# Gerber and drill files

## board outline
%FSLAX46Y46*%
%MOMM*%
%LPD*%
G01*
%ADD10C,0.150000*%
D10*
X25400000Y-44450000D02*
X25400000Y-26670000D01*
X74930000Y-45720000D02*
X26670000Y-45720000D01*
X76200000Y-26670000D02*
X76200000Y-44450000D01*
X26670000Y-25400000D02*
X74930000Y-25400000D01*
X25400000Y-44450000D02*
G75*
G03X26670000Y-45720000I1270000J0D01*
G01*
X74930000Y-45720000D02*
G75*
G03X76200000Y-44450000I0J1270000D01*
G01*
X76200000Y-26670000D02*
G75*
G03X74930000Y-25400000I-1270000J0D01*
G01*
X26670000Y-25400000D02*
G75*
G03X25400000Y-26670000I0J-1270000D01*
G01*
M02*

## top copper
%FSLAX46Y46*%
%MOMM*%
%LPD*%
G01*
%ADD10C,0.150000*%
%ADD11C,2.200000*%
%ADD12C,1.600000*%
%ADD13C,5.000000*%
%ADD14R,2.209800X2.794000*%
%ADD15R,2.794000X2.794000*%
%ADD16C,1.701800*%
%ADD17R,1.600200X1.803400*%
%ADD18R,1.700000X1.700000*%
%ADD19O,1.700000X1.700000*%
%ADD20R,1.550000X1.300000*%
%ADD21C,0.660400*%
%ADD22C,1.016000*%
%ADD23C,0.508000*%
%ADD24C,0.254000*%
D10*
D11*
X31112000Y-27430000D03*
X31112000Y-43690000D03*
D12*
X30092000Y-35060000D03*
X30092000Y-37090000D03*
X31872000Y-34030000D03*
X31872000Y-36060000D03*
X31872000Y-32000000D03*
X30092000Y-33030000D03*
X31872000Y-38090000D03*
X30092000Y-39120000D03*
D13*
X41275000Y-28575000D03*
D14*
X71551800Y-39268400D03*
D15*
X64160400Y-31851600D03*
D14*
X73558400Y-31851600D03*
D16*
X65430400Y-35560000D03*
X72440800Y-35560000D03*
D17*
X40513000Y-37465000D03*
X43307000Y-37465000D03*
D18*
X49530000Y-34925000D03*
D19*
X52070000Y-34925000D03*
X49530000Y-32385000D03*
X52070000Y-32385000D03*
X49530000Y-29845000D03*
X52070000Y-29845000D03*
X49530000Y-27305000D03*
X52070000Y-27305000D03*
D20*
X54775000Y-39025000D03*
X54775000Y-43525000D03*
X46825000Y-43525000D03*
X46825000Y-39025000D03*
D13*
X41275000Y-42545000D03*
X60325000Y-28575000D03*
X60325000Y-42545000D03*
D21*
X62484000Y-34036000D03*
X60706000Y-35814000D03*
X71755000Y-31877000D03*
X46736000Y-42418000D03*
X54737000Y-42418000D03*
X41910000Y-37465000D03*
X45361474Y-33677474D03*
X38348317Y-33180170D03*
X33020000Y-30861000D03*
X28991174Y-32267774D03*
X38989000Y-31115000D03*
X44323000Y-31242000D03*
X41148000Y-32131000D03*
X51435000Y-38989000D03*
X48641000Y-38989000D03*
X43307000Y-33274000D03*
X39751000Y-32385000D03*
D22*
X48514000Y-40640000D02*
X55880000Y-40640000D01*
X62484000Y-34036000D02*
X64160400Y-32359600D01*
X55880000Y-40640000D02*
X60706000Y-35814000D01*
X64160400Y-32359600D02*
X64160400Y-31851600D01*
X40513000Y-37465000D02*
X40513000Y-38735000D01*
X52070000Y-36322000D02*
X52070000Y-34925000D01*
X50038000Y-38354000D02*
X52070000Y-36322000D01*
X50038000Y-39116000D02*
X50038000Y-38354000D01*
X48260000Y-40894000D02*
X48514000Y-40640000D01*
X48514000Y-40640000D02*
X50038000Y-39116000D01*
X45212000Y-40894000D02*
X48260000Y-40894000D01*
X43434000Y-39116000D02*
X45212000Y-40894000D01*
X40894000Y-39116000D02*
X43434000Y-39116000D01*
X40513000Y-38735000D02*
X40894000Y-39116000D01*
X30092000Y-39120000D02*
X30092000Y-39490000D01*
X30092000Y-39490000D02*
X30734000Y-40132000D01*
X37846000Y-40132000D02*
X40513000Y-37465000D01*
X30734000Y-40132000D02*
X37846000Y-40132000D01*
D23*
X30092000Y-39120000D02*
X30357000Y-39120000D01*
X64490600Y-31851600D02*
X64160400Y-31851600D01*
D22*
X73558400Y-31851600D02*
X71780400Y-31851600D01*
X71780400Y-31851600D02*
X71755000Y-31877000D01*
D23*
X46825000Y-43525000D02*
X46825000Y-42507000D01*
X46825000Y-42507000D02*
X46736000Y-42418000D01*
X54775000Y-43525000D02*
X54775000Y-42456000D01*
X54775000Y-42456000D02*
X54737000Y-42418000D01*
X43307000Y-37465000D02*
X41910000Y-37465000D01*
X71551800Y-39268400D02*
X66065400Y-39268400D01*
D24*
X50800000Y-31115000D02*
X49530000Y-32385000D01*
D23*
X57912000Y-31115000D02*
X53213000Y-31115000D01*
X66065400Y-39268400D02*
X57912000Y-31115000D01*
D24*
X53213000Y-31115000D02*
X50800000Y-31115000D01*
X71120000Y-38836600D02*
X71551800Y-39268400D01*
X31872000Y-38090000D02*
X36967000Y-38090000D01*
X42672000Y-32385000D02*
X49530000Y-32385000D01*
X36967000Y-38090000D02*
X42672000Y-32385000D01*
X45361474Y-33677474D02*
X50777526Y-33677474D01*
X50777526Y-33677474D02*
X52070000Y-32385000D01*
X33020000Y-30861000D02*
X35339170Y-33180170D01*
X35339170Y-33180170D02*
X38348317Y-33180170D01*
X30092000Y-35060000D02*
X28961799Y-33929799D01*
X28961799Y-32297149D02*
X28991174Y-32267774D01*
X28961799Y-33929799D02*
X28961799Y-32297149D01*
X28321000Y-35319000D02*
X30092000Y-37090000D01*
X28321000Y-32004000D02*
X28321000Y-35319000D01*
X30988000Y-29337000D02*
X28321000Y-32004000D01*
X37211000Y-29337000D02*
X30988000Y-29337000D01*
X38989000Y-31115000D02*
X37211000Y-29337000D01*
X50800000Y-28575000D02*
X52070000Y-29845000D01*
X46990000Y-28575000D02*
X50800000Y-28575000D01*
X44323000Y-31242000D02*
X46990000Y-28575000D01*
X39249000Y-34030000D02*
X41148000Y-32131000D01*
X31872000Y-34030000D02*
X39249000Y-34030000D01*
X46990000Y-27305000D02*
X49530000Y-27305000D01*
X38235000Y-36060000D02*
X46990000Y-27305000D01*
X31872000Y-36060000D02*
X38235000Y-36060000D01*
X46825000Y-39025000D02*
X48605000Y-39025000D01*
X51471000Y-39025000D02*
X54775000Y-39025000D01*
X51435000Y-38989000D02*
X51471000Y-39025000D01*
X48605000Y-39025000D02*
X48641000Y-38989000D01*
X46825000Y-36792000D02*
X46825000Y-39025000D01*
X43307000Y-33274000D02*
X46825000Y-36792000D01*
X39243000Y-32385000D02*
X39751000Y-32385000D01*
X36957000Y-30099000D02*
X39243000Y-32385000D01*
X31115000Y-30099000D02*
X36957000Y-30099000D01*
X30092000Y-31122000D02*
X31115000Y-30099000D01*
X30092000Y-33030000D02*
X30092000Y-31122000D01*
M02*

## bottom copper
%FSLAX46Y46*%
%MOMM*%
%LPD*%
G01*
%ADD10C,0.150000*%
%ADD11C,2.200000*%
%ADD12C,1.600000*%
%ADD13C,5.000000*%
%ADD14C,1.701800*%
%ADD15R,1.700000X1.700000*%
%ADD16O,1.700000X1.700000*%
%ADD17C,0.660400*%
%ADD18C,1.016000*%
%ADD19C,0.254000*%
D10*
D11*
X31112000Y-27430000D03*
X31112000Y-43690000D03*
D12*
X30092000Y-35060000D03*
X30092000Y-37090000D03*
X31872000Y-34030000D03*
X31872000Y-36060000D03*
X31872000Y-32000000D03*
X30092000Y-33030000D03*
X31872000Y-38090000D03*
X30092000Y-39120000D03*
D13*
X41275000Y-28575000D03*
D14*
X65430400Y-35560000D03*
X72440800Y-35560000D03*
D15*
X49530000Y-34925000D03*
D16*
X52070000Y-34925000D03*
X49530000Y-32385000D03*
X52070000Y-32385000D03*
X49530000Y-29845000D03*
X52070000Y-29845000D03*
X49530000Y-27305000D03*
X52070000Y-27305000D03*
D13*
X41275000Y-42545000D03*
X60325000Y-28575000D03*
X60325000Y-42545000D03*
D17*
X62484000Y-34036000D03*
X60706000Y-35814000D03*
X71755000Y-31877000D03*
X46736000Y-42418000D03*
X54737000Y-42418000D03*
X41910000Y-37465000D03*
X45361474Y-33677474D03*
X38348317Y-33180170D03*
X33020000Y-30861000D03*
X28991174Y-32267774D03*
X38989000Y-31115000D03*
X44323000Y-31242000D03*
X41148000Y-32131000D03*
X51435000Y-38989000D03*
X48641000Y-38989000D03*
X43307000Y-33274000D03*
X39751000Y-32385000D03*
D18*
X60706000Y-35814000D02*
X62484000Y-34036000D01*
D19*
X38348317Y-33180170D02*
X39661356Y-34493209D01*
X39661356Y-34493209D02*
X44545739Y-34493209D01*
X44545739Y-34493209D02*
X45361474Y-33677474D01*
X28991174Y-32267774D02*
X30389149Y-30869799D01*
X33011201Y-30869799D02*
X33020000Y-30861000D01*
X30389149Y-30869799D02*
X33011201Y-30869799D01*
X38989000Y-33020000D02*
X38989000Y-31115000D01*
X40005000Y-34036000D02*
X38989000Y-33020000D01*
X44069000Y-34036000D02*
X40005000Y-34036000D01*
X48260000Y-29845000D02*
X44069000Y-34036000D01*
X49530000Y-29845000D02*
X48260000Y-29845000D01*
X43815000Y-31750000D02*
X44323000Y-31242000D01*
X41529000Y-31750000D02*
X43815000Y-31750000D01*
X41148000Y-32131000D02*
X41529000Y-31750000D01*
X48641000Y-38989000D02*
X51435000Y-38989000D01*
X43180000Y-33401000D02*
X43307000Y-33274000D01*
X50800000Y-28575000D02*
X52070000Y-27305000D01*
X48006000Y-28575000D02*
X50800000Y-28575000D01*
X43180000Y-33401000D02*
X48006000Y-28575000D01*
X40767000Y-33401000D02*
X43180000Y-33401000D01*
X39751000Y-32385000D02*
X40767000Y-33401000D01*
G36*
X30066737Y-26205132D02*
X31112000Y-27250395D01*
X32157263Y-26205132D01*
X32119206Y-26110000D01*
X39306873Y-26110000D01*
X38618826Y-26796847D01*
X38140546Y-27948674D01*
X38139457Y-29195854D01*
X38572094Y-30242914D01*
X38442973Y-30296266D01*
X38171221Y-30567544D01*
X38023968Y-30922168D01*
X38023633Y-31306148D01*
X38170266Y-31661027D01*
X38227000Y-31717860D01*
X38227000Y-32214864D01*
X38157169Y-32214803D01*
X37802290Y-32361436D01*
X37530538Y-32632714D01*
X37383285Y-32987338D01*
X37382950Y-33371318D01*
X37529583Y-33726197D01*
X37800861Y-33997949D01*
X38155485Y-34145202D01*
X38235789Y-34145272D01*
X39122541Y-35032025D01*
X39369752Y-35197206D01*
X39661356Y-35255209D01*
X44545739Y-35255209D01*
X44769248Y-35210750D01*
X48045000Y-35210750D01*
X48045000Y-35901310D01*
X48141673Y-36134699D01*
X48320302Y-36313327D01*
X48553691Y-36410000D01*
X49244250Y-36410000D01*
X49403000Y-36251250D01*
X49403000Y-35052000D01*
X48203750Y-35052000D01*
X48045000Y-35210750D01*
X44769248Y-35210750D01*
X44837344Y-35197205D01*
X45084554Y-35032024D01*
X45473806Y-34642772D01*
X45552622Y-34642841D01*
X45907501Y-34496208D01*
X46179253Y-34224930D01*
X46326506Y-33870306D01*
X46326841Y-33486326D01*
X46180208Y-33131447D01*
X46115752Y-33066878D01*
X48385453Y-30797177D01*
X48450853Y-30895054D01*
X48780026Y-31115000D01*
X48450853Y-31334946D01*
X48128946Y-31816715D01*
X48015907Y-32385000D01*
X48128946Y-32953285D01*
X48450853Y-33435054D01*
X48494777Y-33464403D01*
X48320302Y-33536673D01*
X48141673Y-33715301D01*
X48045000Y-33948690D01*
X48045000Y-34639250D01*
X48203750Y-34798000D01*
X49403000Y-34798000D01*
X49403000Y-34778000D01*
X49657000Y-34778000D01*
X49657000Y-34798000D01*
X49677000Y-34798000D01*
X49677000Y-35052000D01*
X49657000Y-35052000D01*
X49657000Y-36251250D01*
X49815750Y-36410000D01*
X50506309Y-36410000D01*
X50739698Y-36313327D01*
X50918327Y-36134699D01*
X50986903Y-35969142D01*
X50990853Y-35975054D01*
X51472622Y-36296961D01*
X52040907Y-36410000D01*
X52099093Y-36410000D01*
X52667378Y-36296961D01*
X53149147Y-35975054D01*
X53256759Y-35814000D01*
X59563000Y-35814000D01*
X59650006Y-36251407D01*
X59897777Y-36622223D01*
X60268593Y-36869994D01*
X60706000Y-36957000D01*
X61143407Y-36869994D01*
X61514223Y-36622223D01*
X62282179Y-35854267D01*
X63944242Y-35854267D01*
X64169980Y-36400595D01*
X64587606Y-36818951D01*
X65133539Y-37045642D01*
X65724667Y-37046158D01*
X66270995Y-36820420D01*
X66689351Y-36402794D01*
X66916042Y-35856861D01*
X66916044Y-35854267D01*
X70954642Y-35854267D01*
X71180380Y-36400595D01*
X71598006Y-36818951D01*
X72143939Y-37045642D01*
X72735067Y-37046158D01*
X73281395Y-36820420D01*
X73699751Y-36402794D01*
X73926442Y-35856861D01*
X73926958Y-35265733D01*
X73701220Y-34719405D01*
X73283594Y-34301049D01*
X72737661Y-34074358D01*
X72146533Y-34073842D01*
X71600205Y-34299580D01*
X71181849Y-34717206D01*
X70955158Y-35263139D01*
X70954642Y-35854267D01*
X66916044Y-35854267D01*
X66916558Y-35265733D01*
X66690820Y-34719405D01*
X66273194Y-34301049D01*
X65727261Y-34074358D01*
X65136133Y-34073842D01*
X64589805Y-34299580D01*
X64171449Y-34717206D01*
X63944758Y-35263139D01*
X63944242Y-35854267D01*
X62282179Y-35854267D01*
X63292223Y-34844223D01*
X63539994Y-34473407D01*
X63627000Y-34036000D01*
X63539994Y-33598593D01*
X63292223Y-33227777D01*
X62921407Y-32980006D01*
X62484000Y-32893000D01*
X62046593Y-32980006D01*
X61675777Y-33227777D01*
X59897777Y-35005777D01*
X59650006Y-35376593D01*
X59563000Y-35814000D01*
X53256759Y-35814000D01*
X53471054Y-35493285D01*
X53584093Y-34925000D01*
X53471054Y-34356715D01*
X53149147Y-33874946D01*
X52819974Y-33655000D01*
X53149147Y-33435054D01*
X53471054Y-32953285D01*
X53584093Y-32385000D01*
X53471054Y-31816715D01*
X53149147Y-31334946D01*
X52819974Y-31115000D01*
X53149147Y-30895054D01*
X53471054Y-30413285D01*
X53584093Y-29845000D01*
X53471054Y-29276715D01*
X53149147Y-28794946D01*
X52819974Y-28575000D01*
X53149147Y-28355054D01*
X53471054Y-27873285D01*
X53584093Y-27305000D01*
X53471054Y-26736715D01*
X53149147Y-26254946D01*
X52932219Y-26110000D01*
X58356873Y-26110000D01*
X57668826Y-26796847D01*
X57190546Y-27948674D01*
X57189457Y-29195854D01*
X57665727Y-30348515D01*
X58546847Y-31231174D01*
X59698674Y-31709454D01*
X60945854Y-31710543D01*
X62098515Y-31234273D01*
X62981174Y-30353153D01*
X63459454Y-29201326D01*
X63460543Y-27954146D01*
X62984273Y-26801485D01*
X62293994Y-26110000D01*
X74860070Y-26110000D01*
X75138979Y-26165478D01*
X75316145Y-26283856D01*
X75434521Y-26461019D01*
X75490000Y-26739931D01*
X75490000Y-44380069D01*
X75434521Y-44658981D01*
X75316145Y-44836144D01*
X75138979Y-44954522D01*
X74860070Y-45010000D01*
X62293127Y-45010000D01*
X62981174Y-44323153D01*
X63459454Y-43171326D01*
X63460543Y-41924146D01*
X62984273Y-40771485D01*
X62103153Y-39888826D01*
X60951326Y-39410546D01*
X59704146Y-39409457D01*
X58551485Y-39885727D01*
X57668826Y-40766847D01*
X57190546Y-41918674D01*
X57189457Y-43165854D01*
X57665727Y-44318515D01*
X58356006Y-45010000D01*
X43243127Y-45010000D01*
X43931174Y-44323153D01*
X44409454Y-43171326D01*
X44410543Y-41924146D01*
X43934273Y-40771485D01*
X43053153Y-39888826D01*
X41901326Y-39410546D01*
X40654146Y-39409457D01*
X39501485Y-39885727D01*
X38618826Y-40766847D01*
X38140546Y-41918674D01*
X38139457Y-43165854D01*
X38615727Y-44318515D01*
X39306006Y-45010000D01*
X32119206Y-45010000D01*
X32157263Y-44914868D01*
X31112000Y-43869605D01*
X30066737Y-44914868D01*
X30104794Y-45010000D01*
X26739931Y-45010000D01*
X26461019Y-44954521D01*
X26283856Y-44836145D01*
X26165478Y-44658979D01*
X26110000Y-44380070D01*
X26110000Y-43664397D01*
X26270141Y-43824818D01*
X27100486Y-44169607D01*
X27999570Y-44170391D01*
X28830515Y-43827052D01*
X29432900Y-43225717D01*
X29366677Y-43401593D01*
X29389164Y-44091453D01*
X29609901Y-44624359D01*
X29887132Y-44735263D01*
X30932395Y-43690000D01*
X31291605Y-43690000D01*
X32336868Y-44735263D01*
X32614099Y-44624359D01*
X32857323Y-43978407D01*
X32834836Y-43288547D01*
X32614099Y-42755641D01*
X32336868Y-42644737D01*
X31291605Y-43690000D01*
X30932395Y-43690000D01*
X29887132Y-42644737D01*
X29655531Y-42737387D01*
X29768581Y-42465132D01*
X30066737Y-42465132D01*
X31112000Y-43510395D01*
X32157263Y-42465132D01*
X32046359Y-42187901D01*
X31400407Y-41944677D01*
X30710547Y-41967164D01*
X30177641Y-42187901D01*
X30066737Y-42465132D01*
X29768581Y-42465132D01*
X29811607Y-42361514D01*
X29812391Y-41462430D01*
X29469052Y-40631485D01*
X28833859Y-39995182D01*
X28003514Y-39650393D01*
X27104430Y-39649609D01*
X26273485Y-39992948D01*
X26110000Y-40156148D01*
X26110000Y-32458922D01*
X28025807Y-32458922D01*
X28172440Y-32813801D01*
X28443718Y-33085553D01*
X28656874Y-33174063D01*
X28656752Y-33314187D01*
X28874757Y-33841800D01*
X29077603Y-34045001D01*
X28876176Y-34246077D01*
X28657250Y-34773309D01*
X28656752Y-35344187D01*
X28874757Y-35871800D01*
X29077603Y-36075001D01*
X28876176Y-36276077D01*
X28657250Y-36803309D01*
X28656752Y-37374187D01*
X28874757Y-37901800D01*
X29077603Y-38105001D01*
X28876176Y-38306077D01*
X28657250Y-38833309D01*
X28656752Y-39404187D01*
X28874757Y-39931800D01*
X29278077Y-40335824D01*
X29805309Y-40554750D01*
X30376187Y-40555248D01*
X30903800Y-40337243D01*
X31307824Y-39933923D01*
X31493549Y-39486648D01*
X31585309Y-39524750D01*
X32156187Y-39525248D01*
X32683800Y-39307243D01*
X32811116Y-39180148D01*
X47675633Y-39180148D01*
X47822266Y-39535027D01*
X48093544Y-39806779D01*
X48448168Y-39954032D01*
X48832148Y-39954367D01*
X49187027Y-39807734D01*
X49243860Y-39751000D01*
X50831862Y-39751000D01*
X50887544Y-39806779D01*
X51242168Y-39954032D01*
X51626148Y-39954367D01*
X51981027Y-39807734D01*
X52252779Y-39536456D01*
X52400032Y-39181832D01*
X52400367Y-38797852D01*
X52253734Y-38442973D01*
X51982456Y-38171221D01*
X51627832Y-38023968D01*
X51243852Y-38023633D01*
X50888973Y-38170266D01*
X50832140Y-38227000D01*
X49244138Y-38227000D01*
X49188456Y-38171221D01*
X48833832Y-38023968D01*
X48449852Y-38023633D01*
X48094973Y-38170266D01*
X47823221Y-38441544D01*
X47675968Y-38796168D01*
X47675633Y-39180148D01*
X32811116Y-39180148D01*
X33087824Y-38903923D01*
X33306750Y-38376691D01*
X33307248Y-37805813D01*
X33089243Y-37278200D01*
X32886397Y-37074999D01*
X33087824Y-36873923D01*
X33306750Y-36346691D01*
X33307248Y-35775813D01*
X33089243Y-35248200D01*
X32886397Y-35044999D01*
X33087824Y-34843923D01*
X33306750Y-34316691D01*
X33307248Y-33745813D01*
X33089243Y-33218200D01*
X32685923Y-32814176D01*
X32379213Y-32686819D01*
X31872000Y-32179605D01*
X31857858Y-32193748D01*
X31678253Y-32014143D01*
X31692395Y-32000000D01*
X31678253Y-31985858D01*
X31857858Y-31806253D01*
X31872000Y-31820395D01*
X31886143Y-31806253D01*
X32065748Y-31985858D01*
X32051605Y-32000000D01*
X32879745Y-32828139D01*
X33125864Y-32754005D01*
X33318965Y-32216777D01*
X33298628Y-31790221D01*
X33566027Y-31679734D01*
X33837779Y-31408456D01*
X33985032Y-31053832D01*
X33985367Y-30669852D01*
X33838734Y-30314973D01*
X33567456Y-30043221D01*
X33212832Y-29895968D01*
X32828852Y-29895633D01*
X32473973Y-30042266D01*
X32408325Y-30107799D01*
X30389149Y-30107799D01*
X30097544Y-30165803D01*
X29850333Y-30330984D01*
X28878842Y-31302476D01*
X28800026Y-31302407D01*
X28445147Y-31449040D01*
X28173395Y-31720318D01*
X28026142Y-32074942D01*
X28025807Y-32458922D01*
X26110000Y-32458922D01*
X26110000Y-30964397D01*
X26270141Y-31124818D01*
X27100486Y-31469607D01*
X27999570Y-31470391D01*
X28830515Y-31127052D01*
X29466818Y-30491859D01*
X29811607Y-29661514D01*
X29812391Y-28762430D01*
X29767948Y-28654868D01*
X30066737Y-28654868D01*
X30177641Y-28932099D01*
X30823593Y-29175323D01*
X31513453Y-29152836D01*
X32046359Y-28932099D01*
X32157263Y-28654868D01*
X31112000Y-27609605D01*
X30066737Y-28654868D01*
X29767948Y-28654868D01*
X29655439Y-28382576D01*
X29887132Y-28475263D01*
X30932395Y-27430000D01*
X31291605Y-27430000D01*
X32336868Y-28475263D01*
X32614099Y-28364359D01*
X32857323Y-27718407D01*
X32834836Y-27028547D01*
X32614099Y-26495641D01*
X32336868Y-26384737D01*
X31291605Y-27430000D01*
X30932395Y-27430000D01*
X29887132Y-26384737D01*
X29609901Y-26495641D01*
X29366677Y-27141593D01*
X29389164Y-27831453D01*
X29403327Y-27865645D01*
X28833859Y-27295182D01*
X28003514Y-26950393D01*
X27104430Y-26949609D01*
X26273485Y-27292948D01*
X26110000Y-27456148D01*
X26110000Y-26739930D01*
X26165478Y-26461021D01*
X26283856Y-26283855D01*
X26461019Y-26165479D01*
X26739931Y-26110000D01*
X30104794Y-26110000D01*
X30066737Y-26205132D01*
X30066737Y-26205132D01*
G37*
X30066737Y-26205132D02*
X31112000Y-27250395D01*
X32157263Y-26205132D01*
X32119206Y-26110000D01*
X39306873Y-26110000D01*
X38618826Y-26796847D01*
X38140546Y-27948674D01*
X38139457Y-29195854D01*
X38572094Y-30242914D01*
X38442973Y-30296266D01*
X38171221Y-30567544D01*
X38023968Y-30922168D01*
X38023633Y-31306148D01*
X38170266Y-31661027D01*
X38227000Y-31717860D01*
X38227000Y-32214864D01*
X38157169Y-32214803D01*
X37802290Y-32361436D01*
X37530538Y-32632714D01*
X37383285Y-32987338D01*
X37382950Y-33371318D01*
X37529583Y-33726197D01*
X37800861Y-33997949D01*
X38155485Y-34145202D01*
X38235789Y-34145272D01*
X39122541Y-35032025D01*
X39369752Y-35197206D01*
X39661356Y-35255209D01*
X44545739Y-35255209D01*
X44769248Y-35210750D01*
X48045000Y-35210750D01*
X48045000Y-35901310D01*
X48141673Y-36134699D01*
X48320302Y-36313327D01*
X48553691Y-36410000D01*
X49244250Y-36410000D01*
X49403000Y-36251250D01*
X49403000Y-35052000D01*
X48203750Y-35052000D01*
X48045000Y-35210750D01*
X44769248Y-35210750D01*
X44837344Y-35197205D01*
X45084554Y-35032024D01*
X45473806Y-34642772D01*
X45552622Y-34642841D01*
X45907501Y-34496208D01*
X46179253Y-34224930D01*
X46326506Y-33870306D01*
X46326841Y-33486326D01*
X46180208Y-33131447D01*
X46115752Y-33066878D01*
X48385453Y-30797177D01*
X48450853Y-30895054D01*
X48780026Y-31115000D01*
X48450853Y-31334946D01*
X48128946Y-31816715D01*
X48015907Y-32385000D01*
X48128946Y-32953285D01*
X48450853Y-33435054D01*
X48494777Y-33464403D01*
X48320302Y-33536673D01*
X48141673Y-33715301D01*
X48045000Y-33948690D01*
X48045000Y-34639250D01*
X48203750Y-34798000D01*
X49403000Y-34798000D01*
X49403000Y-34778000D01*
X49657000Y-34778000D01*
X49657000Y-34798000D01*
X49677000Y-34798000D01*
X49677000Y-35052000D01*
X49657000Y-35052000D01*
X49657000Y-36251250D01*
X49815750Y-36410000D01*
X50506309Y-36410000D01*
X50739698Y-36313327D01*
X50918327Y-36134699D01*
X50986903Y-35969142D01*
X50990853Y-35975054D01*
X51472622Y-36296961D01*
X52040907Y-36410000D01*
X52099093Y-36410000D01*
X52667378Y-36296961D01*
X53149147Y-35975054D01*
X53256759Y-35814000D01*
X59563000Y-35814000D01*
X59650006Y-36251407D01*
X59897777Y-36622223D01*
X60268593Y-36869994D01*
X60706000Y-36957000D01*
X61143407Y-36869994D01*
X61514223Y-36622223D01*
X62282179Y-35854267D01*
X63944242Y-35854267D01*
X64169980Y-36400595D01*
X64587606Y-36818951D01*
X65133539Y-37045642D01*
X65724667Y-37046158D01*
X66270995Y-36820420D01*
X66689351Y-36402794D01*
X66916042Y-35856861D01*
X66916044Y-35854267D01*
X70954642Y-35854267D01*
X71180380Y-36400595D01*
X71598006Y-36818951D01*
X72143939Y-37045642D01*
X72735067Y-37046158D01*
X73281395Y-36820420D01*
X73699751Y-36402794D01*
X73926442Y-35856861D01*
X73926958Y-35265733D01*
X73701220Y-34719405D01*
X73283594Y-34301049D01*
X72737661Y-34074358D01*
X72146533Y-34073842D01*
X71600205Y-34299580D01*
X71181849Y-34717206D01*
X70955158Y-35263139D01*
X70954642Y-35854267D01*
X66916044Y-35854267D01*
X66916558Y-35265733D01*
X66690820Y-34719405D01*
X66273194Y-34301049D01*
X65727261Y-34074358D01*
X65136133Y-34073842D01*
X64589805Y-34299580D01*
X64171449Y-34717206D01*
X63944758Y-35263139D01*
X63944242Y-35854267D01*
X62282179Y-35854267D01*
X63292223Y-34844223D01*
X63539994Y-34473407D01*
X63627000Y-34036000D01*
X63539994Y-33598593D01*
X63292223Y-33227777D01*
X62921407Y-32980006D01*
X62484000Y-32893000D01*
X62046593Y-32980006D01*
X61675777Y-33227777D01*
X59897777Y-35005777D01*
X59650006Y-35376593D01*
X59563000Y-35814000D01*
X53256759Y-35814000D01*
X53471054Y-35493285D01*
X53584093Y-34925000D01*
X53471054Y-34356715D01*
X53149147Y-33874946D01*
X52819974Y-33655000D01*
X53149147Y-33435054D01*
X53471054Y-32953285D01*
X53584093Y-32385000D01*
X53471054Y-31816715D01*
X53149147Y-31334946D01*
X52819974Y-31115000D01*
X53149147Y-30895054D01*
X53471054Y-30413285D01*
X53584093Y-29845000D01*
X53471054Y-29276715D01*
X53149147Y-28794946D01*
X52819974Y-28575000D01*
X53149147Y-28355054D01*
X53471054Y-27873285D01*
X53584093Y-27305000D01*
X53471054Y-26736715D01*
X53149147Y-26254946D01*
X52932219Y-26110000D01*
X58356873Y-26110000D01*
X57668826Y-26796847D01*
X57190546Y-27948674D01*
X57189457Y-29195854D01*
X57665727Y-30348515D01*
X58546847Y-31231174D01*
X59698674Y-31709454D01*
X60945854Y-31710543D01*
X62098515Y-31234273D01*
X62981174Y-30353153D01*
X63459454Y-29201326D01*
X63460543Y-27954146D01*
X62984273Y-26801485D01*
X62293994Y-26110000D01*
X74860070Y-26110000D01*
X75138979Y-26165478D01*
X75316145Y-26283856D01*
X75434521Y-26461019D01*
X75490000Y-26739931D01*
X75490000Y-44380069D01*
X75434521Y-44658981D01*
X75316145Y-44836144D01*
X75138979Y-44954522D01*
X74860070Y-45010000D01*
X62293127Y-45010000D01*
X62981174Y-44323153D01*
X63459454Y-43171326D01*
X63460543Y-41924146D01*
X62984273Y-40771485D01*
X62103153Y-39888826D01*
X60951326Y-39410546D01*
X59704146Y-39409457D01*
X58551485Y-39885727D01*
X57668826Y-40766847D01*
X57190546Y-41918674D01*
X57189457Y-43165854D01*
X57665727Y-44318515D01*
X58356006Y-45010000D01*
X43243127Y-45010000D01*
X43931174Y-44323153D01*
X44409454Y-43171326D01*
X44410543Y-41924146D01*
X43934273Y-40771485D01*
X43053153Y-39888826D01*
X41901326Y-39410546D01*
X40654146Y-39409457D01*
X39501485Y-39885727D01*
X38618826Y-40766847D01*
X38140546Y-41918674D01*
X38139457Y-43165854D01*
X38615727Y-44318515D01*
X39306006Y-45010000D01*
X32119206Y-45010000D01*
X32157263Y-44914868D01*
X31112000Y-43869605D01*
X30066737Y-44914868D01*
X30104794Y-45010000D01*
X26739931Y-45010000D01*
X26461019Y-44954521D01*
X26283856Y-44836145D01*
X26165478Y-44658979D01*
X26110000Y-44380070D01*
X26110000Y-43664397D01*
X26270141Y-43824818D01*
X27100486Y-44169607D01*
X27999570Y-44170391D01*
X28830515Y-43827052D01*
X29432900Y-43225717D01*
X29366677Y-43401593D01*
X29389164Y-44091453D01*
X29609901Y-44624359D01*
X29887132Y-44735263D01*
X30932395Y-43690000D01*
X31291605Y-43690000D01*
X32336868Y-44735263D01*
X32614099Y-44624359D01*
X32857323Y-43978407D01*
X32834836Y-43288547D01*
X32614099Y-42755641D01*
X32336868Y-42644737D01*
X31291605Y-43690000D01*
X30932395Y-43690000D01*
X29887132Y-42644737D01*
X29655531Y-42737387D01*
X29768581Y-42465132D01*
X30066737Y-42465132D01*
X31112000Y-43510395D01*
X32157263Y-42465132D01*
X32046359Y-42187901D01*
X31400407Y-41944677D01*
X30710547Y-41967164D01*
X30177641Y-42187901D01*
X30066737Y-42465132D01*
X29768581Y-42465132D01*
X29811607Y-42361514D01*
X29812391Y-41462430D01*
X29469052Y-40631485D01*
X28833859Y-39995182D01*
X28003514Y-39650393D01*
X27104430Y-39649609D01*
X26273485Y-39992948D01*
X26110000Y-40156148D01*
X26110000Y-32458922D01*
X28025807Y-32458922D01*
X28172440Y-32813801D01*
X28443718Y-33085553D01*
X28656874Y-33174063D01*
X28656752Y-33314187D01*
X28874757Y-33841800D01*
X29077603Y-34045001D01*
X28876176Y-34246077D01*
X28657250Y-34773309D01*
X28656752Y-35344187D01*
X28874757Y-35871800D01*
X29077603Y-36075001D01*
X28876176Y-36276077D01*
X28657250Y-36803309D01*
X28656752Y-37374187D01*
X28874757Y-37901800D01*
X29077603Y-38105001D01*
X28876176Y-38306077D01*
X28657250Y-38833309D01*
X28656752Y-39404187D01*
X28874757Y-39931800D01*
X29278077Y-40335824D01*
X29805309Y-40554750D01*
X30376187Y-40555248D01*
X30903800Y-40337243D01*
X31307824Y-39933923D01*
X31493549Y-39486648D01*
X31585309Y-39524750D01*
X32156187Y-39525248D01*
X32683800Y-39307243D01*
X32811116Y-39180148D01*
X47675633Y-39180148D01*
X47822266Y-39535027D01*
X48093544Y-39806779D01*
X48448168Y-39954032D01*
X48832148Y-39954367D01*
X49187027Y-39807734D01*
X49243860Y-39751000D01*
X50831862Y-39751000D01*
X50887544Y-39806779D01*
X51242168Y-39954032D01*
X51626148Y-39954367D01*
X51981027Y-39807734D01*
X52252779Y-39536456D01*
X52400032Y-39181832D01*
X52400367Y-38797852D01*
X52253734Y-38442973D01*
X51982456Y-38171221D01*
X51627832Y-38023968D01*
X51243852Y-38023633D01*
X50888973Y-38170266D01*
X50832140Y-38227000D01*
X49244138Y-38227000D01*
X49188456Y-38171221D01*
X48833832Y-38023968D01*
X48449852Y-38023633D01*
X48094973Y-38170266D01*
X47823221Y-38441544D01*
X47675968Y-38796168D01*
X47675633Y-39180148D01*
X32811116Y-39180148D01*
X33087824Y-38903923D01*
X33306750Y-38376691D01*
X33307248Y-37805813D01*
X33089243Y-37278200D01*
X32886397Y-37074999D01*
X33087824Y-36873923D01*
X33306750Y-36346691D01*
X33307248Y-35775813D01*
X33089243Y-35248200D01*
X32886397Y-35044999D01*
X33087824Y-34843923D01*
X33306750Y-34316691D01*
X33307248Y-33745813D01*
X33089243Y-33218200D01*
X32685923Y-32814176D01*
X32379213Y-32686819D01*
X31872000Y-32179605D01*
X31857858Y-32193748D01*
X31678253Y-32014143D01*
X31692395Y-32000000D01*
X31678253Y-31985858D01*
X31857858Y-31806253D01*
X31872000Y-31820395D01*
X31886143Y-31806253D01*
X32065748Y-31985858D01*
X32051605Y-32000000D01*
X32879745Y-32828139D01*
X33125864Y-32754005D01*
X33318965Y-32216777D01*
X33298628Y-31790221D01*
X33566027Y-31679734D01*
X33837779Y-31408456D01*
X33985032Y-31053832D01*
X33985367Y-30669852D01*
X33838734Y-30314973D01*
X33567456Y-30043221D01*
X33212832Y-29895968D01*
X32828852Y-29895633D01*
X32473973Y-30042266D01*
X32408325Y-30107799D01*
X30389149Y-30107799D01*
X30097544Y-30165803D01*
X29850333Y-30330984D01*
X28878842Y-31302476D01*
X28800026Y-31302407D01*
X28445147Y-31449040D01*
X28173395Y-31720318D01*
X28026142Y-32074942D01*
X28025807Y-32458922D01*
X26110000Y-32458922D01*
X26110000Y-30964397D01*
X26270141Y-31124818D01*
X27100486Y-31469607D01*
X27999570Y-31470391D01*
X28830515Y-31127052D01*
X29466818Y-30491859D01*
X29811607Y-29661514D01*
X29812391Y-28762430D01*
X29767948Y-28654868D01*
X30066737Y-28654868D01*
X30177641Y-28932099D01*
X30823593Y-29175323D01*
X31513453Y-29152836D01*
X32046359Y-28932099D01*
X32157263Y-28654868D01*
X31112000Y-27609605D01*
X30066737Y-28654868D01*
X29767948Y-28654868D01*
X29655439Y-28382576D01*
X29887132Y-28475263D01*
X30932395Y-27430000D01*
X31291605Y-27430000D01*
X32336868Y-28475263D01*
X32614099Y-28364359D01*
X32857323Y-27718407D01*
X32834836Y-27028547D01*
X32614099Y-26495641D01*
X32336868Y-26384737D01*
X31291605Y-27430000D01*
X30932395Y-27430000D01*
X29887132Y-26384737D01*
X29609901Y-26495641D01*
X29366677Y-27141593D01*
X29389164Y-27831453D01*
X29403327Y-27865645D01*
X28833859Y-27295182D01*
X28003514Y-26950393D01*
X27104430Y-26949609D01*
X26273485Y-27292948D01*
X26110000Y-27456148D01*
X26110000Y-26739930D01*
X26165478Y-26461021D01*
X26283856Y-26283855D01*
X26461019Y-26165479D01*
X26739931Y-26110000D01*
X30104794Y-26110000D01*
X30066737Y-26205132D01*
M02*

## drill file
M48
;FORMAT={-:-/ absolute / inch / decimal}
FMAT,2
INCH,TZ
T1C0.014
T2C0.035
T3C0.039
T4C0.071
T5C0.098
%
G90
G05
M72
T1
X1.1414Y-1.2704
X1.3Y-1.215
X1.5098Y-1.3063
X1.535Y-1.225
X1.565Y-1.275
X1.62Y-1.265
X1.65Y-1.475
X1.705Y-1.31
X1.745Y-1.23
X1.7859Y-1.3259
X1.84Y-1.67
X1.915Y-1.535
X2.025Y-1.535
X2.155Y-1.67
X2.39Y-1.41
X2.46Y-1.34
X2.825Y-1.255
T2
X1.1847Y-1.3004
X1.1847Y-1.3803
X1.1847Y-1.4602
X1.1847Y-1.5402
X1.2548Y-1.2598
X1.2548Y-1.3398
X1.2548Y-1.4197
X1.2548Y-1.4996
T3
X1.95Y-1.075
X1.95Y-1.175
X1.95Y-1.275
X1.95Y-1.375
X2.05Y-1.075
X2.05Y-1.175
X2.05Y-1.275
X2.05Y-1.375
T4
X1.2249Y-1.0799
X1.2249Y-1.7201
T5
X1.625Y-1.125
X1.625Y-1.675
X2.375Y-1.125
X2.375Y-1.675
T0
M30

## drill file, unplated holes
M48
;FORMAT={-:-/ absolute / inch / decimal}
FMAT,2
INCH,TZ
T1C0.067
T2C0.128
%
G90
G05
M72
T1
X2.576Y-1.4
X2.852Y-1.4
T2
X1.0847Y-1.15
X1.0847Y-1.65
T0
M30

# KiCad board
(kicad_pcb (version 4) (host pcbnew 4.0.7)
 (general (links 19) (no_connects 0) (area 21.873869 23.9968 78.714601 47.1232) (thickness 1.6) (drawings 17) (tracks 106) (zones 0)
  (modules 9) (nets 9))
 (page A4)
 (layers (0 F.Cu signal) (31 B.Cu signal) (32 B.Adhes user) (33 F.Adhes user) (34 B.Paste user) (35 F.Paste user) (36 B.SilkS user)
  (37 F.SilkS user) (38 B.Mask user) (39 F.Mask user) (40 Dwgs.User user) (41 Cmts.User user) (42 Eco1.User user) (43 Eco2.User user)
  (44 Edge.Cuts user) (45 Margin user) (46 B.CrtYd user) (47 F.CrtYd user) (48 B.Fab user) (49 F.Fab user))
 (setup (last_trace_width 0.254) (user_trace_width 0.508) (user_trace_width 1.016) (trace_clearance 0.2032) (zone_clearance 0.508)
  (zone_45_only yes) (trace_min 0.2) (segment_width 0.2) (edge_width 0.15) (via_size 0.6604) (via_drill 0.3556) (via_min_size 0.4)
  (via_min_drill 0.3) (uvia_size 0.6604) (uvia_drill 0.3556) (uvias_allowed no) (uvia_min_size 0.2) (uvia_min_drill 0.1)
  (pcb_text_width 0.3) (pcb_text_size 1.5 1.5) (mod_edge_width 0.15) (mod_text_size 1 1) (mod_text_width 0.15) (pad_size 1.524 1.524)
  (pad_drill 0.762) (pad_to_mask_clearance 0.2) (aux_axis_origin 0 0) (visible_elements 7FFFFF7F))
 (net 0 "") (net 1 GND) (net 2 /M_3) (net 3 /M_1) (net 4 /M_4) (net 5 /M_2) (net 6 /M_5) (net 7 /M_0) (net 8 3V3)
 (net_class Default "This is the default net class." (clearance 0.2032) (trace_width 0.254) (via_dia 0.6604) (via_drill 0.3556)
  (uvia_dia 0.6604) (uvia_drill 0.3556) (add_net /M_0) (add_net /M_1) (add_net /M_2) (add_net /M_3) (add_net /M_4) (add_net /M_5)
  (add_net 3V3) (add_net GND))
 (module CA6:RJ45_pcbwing (layer F.Cu) (at 29.972 35.56 270)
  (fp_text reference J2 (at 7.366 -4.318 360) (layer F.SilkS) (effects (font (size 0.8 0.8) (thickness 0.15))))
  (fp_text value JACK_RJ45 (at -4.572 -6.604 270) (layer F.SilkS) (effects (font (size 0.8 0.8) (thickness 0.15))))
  (pad 8 thru_hole circle (at -8.13 -1.14 270) (size 2.2 2.2) (drill 1.8) (layers *.Cu *.Mask F.SilkS) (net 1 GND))
  (pad 8 thru_hole circle (at 8.13 -1.14 270) (size 2.2 2.2) (drill 1.8) (layers *.Cu *.Mask F.SilkS) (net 1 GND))
  (pad "" np_thru_hole circle (at -6.35 2.42 270) (size 3.25 3.25) (drill 3.25) (layers *.Cu *.Mask F.SilkS))
  (pad "" np_thru_hole circle (at 6.35 2.42 270) (size 3.25 3.25) (drill 3.25) (layers *.Cu *.Mask F.SilkS))
  (pad 5 thru_hole circle (at -0.5 -0.12 270) (size 1.6 1.6) (drill 0.89) (layers *.Cu *.Mask F.SilkS) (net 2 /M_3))
  (pad 3 thru_hole circle (at 1.53 -0.12 270) (size 1.6 1.6) (drill 0.89) (layers *.Cu *.Mask F.SilkS) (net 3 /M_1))
  (pad 6 thru_hole circle (at -1.53 -1.9 270) (size 1.6 1.6) (drill 0.89) (layers *.Cu *.Mask F.SilkS) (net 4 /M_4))
  (pad 4 thru_hole circle (at 0.5 -1.9 270) (size 1.6 1.6) (drill 0.89) (layers *.Cu *.Mask F.SilkS) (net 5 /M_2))
  (pad 8 thru_hole circle (at -3.56 -1.9 270) (size 1.6 1.6) (drill 0.89) (layers *.Cu *.Mask F.SilkS) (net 1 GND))
  (pad 7 thru_hole circle (at -2.53 -0.12 270) (size 1.6 1.6) (drill 0.89) (layers *.Cu *.Mask F.SilkS) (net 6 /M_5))
  (pad 2 thru_hole circle (at 2.53 -1.9 270) (size 1.6 1.6) (drill 0.89) (layers *.Cu *.Mask F.SilkS) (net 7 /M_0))
  (pad 1 thru_hole circle (at 3.56 -0.12 270) (size 1.6 1.6) (drill 0.89) (layers *.Cu *.Mask F.SilkS) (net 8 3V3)))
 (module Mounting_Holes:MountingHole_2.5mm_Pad (layer F.Cu) (at 41.275 28.575)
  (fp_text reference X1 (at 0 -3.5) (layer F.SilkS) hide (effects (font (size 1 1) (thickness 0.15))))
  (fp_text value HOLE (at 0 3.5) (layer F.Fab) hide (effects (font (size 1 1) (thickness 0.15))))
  (pad 1 thru_hole circle (at 0 0) (size 5 5) (drill 2.5) (layers *.Cu *.Mask)))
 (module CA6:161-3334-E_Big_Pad (layer F.Cu) (at 75.946 35.56 180)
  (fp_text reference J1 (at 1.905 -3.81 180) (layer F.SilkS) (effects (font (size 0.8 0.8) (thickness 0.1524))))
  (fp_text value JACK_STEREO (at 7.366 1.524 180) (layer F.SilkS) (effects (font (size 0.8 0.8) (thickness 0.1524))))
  (pad 1 smd rect (at 4.3942 -3.7084 180) (size 2.2098 2.794) (layers F.Cu F.Paste F.Mask) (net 7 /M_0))
  (pad 2 smd rect (at 11.7856 3.7084 180) (size 2.794 2.794) (layers F.Cu F.Paste F.Mask) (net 8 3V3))
  (pad 3 smd rect (at 2.3876 3.7084 180) (size 2.2098 2.794) (layers F.Cu F.Paste F.Mask) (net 1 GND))
  (pad "" np_thru_hole circle (at 10.5156 0 90) (size 1.7018 1.7018) (drill 1.7) (layers *.Cu *.Mask F.SilkS))
  (pad "" np_thru_hole circle (at 3.5052 0 90) (size 1.7018 1.7018) (drill 1.7) (layers *.Cu *.Mask F.SilkS)))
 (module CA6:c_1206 (layer F.Cu) (at 41.91 37.465 180)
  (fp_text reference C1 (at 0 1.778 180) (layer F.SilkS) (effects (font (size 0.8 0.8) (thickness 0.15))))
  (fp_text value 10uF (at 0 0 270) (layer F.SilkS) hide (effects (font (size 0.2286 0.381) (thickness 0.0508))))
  (pad 1 smd rect (at 1.397 0 180) (size 1.6002 1.8034) (layers F.Cu F.Paste F.Mask) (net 8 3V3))
  (pad 2 smd rect (at -1.397 0 180) (size 1.6002 1.8034) (layers F.Cu F.Paste F.Mask) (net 1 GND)))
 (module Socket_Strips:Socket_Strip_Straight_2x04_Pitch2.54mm (layer F.Cu) (at 49.53 34.925 180)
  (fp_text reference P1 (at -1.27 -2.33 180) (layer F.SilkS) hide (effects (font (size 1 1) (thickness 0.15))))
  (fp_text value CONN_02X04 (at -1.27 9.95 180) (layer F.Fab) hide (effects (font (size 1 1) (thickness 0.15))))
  (pad 1 thru_hole rect (at 0 0 180) (size 1.7 1.7) (drill 1) (layers *.Cu *.Mask) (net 1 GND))
  (pad 2 thru_hole oval (at -2.54 0 180) (size 1.7 1.7) (drill 1) (layers *.Cu *.Mask) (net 8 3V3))
  (pad 3 thru_hole oval (at 0 2.54 180) (size 1.7 1.7) (drill 1) (layers *.Cu *.Mask) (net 7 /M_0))
  (pad 4 thru_hole oval (at -2.54 2.54 180) (size 1.7 1.7) (drill 1) (layers *.Cu *.Mask) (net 2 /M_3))
  (pad 5 thru_hole oval (at 0 5.08 180) (size 1.7 1.7) (drill 1) (layers *.Cu *.Mask) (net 3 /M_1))
  (pad 6 thru_hole oval (at -2.54 5.08 180) (size 1.7 1.7) (drill 1) (layers *.Cu *.Mask) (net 4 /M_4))
  (pad 7 thru_hole oval (at 0 7.62 180) (size 1.7 1.7) (drill 1) (layers *.Cu *.Mask) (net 5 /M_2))
  (pad 8 thru_hole oval (at -2.54 7.62 180) (size 1.7 1.7) (drill 1) (layers *.Cu *.Mask) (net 6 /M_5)))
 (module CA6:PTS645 (layer F.Cu) (at 50.8 41.275 180)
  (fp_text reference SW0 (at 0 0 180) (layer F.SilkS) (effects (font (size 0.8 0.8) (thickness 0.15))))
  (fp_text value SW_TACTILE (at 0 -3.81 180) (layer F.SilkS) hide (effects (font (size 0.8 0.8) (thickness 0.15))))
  (pad 3 smd rect (at -3.975 2.25 180) (size 1.55 1.3) (layers F.Cu F.Paste F.Mask) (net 6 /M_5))
  (pad 1 smd rect (at -3.975 -2.25 180) (size 1.55 1.3) (layers F.Cu F.Paste F.Mask) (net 1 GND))
  (pad 2 smd rect (at 3.975 -2.25 180) (size 1.55 1.3) (layers F.Cu F.Paste F.Mask) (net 1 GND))
  (pad 4 smd rect (at 3.975 2.25 180) (size 1.55 1.3) (layers F.Cu F.Paste F.Mask) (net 6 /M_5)))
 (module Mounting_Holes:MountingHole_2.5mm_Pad (layer F.Cu) (at 41.275 42.545)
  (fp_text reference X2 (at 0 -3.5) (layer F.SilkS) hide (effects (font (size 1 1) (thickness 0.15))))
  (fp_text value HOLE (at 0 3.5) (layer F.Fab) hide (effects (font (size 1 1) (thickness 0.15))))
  (pad 1 thru_hole circle (at 0 0) (size 5 5) (drill 2.5) (layers *.Cu *.Mask)))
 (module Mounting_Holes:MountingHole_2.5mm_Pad (layer F.Cu) (at 60.325 28.575)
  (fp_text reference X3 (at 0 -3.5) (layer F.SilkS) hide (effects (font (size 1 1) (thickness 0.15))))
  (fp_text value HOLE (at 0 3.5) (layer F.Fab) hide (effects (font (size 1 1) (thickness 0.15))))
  (pad 1 thru_hole circle (at 0 0) (size 5 5) (drill 2.5) (layers *.Cu *.Mask)))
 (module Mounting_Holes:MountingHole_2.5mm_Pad (layer F.Cu) (at 60.325 42.545)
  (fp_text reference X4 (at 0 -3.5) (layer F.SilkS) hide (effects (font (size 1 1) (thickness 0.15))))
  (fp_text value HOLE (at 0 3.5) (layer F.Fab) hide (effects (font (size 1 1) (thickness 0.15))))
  (pad 1 thru_hole circle (at 0 0) (size 5 5) (drill 2.5) (layers *.Cu *.Mask)))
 (gr_line (start 25.4 44.45) (end 25.4 26.67) (angle 90) (layer Edge.Cuts) (width 0.15))
 (gr_line (start 74.93 45.72) (end 26.67 45.72) (angle 90) (layer Edge.Cuts) (width 0.15))
 (gr_line (start 76.2 26.67) (end 76.2 44.45) (angle 90) (layer Edge.Cuts) (width 0.15))
 (gr_line (start 26.67 25.4) (end 74.93 25.4) (angle 90) (layer Edge.Cuts) (width 0.15))
 (gr_arc (start 26.67 44.45) (end 26.67 45.72) (angle 90) (layer Edge.Cuts) (width 0.15))
 (gr_arc (start 74.93 44.45) (end 76.2 44.45) (angle 90) (layer Edge.Cuts) (width 0.15))
 (gr_arc (start 74.93 26.67) (end 74.93 25.4) (angle 90) (layer Edge.Cuts) (width 0.15))
 (gr_arc (start 26.67 26.67) (end 25.4 26.67) (angle 90) (layer Edge.Cuts) (width 0.15))
 (segment (start 48.514 40.64) (end 55.88 40.64) (width 1.016) (layer F.Cu) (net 8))
 (segment (start 62.484 34.036) (end 64.1604 32.3596) (width 1.016) (layer F.Cu) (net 8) (status 20))
 (via (at 62.484 34.036) (size 0.6604) (drill 0.3556) (layers F.Cu B.Cu) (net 8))
 (segment (start 60.706 35.814) (end 62.484 34.036) (width 1.016) (layer B.Cu) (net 8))
 (via (at 60.706 35.814) (size 0.6604) (drill 0.3556) (layers F.Cu B.Cu) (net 8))
 (segment (start 55.88 40.64) (end 60.706 35.814) (width 1.016) (layer F.Cu) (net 8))
 (segment (start 64.1604 32.3596) (end 64.1604 31.8516) (width 1.016) (layer F.Cu) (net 8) (status 30))
 (segment (start 40.513 37.465) (end 40.513 38.735) (width 1.016) (layer F.Cu) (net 8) (status 10))
 (segment (start 52.07 36.322) (end 52.07 34.925) (width 1.016) (layer F.Cu) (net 8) (status 20))
 (segment (start 50.038 38.354) (end 52.07 36.322) (width 1.016) (layer F.Cu) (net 8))
 (segment (start 50.038 39.116) (end 50.038 38.354) (width 1.016) (layer F.Cu) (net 8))
 (segment (start 48.26 40.894) (end 48.514 40.64) (width 1.016) (layer F.Cu) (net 8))
 (segment (start 48.514 40.64) (end 50.038 39.116) (width 1.016) (layer F.Cu) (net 8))
 (segment (start 45.212 40.894) (end 48.26 40.894) (width 1.016) (layer F.Cu) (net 8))
 (segment (start 43.434 39.116) (end 45.212 40.894) (width 1.016) (layer F.Cu) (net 8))
 (segment (start 40.894 39.116) (end 43.434 39.116) (width 1.016) (layer F.Cu) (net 8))
 (segment (start 40.513 38.735) (end 40.894 39.116) (width 1.016) (layer F.Cu) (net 8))
 (segment (start 30.092 39.12) (end 30.092 39.49) (width 1.016) (layer F.Cu) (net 8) (status 30))
 (segment (start 30.092 39.49) (end 30.734 40.132) (width 1.016) (layer F.Cu) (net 8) (status 10))
 (segment (start 37.846 40.132) (end 40.513 37.465) (width 1.016) (layer F.Cu) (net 8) (status 20))
 (segment (start 30.734 40.132) (end 37.846 40.132) (width 1.016) (layer F.Cu) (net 8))
 (segment (start 30.092 39.12) (end 30.357 39.12) (width 0.508) (layer F.Cu) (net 8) (status 30))
 (segment (start 64.4906 31.8516) (end 64.1604 31.8516) (width 0.508) (layer F.Cu) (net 8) (status 30))
 (segment (start 73.5584 31.8516) (end 71.7804 31.8516) (width 1.016) (layer F.Cu) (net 1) (status 10))
 (via (at 71.755 31.877) (size 0.6604) (drill 0.3556) (layers F.Cu B.Cu) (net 1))
 (segment (start 71.7804 31.8516) (end 71.755 31.877) (width 1.016) (layer F.Cu) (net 1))
 (segment (start 46.825 43.525) (end 46.825 42.507) (width 0.508) (layer F.Cu) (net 1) (status 10))
 (via (at 46.736 42.418) (size 0.6604) (drill 0.3556) (layers F.Cu B.Cu) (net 1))
 (segment (start 46.825 42.507) (end 46.736 42.418) (width 0.508) (layer F.Cu) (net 1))
 (segment (start 54.775 43.525) (end 54.775 42.456) (width 0.508) (layer F.Cu) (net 1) (status 10))
 (via (at 54.737 42.418) (size 0.6604) (drill 0.3556) (layers F.Cu B.Cu) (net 1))
 (segment (start 54.775 42.456) (end 54.737 42.418) (width 0.508) (layer F.Cu) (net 1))
 (segment (start 43.307 37.465) (end 41.91 37.465) (width 0.508) (layer F.Cu) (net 1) (status 10))
 (via (at 41.91 37.465) (size 0.6604) (drill 0.3556) (layers F.Cu B.Cu) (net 1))
 (segment (start 71.5518 39.2684) (end 66.0654 39.2684) (width 0.508) (layer F.Cu) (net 7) (status 10))
 (segment (start 50.8 31.115) (end 49.53 32.385) (width 0.254) (layer F.Cu) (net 7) (status 20))
 (segment (start 57.912 31.115) (end 53.213 31.115) (width 0.508) (layer F.Cu) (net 7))
 (segment (start 66.0654 39.2684) (end 57.912 31.115) (width 0.508) (layer F.Cu) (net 7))
 (segment (start 53.213 31.115) (end 50.8 31.115) (width 0.254) (layer F.Cu) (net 7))
 (segment (start 71.12 38.8366) (end 71.5518 39.2684) (width 0.254) (layer F.Cu) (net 7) (status 30))
 (segment (start 31.872 38.09) (end 36.967 38.09) (width 0.254) (layer F.Cu) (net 7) (status 10))
 (segment (start 42.672 32.385) (end 49.53 32.385) (width 0.254) (layer F.Cu) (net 7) (status 20))
 (segment (start 36.967 38.09) (end 42.672 32.385) (width 0.254) (layer F.Cu) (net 7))
 (segment (start 45.361474 33.677474) (end 50.777526 33.677474) (width 0.254) (layer F.Cu) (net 2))
 (segment (start 50.777526 33.677474) (end 52.07 32.385) (width 0.254) (layer F.Cu) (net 2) (status 20))
 (segment (start 38.348317 33.18017) (end 39.661356 34.493209) (width 0.254) (layer B.Cu) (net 2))
 (segment (start 39.661356 34.493209) (end 44.545739 34.493209) (width 0.254) (layer B.Cu) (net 2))
 (segment (start 44.545739 34.493209) (end 45.361474 33.677474) (width 0.254) (layer B.Cu) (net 2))
 (via (at 45.361474 33.677474) (size 0.6604) (drill 0.3556) (layers F.Cu B.Cu) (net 2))
 (segment (start 33.02 30.861) (end 35.33917 33.18017) (width 0.254) (layer F.Cu) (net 2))
 (segment (start 35.33917 33.18017) (end 38.348317 33.18017) (width 0.254) (layer F.Cu) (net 2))
 (via (at 38.348317 33.18017) (size 0.6604) (drill 0.3556) (layers F.Cu B.Cu) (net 2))
 (segment (start 28.991174 32.267774) (end 30.389149 30.869799) (width 0.254) (layer B.Cu) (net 2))
 (segment (start 33.011201 30.869799) (end 33.02 30.861) (width 0.254) (layer B.Cu) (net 2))
 (segment (start 30.389149 30.869799) (end 33.011201 30.869799) (width 0.254) (layer B.Cu) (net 2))
 (via (at 33.02 30.861) (size 0.6604) (drill 0.3556) (layers F.Cu B.Cu) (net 2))
 (segment (start 30.092 35.06) (end 28.961799 33.929799) (width 0.254) (layer F.Cu) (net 2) (status 10))
 (segment (start 28.961799 32.297149) (end 28.991174 32.267774) (width 0.254) (layer F.Cu) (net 2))
 (via (at 28.991174 32.267774) (size 0.6604) (drill 0.3556) (layers F.Cu B.Cu) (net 2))
 (segment (start 28.961799 33.929799) (end 28.961799 32.297149) (width 0.254) (layer F.Cu) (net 2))
 (segment (start 28.321 35.319) (end 30.092 37.09) (width 0.254) (layer F.Cu) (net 3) (status 20))
 (segment (start 28.321 32.004) (end 28.321 35.319) (width 0.254) (layer F.Cu) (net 3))
 (segment (start 30.988 29.337) (end 28.321 32.004) (width 0.254) (layer F.Cu) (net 3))
 (segment (start 37.211 29.337) (end 30.988 29.337) (width 0.254) (layer F.Cu) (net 3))
 (segment (start 38.989 31.115) (end 37.211 29.337) (width 0.254) (layer F.Cu) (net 3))
 (via (at 38.989 31.115) (size 0.6604) (drill 0.3556) (layers F.Cu B.Cu) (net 3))
 (segment (start 38.989 33.02) (end 38.989 31.115) (width 0.254) (layer B.Cu) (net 3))
 (segment (start 40.005 34.036) (end 38.989 33.02) (width 0.254) (layer B.Cu) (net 3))
 (segment (start 44.069 34.036) (end 40.005 34.036) (width 0.254) (layer B.Cu) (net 3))
 (segment (start 48.26 29.845) (end 44.069 34.036) (width 0.254) (layer B.Cu) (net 3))
 (segment (start 49.53 29.845) (end 48.26 29.845) (width 0.254) (layer B.Cu) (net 3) (status 10))
 (segment (start 50.8 28.575) (end 52.07 29.845) (width 0.254) (layer F.Cu) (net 4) (status 20))
 (segment (start 46.99 28.575) (end 50.8 28.575) (width 0.254) (layer F.Cu) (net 4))
 (segment (start 44.323 31.242) (end 46.99 28.575) (width 0.254) (layer F.Cu) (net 4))
 (via (at 44.323 31.242) (size 0.6604) (drill 0.3556) (layers F.Cu B.Cu) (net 4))
 (segment (start 43.815 31.75) (end 44.323 31.242) (width 0.254) (layer B.Cu) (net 4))
 (segment (start 41.529 31.75) (end 43.815 31.75) (width 0.254) (layer B.Cu) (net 4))
 (segment (start 41.148 32.131) (end 41.529 31.75) (width 0.254) (layer B.Cu) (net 4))
 (via (at 41.148 32.131) (size 0.6604) (drill 0.3556) (layers F.Cu B.Cu) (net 4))
 (segment (start 39.249 34.03) (end 41.148 32.131) (width 0.254) (layer F.Cu) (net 4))
 (segment (start 31.872 34.03) (end 39.249 34.03) (width 0.254) (layer F.Cu) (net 4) (status 10))
 (segment (start 46.99 27.305) (end 49.53 27.305) (width 0.254) (layer F.Cu) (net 5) (status 20))
 (segment (start 38.235 36.06) (end 46.99 27.305) (width 0.254) (layer F.Cu) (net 5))
 (segment (start 31.872 36.06) (end 38.235 36.06) (width 0.254) (layer F.Cu) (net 5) (status 10))
 (segment (start 46.825 39.025) (end 48.605 39.025) (width 0.254) (layer F.Cu) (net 6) (status 10))
 (segment (start 51.471 39.025) (end 54.775 39.025) (width 0.254) (layer F.Cu) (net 6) (status 20))
 (segment (start 51.435 38.989) (end 51.471 39.025) (width 0.254) (layer F.Cu) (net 6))
 (via (at 51.435 38.989) (size 0.6604) (drill 0.3556) (layers F.Cu B.Cu) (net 6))
 (segment (start 48.641 38.989) (end 51.435 38.989) (width 0.254) (layer B.Cu) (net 6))
 (via (at 48.641 38.989) (size 0.6604) (drill 0.3556) (layers F.Cu B.Cu) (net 6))
 (segment (start 48.605 39.025) (end 48.641 38.989) (width 0.254) (layer F.Cu) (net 6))
 (segment (start 46.825 36.792) (end 46.825 39.025) (width 0.254) (layer F.Cu) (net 6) (status 20))
 (segment (start 43.307 33.274) (end 46.825 36.792) (width 0.254) (layer F.Cu) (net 6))
 (via (at 43.307 33.274) (size 0.6604) (drill 0.3556) (layers F.Cu B.Cu) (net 6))
 (segment (start 43.18 33.401) (end 43.307 33.274) (width 0.254) (layer B.Cu) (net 6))
 (segment (start 50.8 28.575) (end 52.07 27.305) (width 0.254) (layer B.Cu) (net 6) (status 20))
 (segment (start 48.006 28.575) (end 50.8 28.575) (width 0.254) (layer B.Cu) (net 6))
 (segment (start 43.18 33.401) (end 48.006 28.575) (width 0.254) (layer B.Cu) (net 6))
 (segment (start 40.767 33.401) (end 43.18 33.401) (width 0.254) (layer B.Cu) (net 6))
 (segment (start 39.751 32.385) (end 40.767 33.401) (width 0.254) (layer B.Cu) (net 6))
 (via (at 39.751 32.385) (size 0.6604) (drill 0.3556) (layers F.Cu B.Cu) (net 6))
 (segment (start 39.243 32.385) (end 39.751 32.385) (width 0.254) (layer F.Cu) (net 6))
 (segment (start 36.957 30.099) (end 39.243 32.385) (width 0.254) (layer F.Cu) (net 6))
 (segment (start 31.115 30.099) (end 36.957 30.099) (width 0.254) (layer F.Cu) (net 6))
 (segment (start 30.092 31.122) (end 31.115 30.099) (width 0.254) (layer F.Cu) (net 6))
 (segment (start 30.092 33.03) (end 30.092 31.122) (width 0.254) (layer F.Cu) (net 6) (status 10))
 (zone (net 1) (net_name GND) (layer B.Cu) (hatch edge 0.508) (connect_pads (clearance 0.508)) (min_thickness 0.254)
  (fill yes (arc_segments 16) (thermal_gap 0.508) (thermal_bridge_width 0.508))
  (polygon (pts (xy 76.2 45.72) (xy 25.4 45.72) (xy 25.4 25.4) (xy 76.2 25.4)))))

